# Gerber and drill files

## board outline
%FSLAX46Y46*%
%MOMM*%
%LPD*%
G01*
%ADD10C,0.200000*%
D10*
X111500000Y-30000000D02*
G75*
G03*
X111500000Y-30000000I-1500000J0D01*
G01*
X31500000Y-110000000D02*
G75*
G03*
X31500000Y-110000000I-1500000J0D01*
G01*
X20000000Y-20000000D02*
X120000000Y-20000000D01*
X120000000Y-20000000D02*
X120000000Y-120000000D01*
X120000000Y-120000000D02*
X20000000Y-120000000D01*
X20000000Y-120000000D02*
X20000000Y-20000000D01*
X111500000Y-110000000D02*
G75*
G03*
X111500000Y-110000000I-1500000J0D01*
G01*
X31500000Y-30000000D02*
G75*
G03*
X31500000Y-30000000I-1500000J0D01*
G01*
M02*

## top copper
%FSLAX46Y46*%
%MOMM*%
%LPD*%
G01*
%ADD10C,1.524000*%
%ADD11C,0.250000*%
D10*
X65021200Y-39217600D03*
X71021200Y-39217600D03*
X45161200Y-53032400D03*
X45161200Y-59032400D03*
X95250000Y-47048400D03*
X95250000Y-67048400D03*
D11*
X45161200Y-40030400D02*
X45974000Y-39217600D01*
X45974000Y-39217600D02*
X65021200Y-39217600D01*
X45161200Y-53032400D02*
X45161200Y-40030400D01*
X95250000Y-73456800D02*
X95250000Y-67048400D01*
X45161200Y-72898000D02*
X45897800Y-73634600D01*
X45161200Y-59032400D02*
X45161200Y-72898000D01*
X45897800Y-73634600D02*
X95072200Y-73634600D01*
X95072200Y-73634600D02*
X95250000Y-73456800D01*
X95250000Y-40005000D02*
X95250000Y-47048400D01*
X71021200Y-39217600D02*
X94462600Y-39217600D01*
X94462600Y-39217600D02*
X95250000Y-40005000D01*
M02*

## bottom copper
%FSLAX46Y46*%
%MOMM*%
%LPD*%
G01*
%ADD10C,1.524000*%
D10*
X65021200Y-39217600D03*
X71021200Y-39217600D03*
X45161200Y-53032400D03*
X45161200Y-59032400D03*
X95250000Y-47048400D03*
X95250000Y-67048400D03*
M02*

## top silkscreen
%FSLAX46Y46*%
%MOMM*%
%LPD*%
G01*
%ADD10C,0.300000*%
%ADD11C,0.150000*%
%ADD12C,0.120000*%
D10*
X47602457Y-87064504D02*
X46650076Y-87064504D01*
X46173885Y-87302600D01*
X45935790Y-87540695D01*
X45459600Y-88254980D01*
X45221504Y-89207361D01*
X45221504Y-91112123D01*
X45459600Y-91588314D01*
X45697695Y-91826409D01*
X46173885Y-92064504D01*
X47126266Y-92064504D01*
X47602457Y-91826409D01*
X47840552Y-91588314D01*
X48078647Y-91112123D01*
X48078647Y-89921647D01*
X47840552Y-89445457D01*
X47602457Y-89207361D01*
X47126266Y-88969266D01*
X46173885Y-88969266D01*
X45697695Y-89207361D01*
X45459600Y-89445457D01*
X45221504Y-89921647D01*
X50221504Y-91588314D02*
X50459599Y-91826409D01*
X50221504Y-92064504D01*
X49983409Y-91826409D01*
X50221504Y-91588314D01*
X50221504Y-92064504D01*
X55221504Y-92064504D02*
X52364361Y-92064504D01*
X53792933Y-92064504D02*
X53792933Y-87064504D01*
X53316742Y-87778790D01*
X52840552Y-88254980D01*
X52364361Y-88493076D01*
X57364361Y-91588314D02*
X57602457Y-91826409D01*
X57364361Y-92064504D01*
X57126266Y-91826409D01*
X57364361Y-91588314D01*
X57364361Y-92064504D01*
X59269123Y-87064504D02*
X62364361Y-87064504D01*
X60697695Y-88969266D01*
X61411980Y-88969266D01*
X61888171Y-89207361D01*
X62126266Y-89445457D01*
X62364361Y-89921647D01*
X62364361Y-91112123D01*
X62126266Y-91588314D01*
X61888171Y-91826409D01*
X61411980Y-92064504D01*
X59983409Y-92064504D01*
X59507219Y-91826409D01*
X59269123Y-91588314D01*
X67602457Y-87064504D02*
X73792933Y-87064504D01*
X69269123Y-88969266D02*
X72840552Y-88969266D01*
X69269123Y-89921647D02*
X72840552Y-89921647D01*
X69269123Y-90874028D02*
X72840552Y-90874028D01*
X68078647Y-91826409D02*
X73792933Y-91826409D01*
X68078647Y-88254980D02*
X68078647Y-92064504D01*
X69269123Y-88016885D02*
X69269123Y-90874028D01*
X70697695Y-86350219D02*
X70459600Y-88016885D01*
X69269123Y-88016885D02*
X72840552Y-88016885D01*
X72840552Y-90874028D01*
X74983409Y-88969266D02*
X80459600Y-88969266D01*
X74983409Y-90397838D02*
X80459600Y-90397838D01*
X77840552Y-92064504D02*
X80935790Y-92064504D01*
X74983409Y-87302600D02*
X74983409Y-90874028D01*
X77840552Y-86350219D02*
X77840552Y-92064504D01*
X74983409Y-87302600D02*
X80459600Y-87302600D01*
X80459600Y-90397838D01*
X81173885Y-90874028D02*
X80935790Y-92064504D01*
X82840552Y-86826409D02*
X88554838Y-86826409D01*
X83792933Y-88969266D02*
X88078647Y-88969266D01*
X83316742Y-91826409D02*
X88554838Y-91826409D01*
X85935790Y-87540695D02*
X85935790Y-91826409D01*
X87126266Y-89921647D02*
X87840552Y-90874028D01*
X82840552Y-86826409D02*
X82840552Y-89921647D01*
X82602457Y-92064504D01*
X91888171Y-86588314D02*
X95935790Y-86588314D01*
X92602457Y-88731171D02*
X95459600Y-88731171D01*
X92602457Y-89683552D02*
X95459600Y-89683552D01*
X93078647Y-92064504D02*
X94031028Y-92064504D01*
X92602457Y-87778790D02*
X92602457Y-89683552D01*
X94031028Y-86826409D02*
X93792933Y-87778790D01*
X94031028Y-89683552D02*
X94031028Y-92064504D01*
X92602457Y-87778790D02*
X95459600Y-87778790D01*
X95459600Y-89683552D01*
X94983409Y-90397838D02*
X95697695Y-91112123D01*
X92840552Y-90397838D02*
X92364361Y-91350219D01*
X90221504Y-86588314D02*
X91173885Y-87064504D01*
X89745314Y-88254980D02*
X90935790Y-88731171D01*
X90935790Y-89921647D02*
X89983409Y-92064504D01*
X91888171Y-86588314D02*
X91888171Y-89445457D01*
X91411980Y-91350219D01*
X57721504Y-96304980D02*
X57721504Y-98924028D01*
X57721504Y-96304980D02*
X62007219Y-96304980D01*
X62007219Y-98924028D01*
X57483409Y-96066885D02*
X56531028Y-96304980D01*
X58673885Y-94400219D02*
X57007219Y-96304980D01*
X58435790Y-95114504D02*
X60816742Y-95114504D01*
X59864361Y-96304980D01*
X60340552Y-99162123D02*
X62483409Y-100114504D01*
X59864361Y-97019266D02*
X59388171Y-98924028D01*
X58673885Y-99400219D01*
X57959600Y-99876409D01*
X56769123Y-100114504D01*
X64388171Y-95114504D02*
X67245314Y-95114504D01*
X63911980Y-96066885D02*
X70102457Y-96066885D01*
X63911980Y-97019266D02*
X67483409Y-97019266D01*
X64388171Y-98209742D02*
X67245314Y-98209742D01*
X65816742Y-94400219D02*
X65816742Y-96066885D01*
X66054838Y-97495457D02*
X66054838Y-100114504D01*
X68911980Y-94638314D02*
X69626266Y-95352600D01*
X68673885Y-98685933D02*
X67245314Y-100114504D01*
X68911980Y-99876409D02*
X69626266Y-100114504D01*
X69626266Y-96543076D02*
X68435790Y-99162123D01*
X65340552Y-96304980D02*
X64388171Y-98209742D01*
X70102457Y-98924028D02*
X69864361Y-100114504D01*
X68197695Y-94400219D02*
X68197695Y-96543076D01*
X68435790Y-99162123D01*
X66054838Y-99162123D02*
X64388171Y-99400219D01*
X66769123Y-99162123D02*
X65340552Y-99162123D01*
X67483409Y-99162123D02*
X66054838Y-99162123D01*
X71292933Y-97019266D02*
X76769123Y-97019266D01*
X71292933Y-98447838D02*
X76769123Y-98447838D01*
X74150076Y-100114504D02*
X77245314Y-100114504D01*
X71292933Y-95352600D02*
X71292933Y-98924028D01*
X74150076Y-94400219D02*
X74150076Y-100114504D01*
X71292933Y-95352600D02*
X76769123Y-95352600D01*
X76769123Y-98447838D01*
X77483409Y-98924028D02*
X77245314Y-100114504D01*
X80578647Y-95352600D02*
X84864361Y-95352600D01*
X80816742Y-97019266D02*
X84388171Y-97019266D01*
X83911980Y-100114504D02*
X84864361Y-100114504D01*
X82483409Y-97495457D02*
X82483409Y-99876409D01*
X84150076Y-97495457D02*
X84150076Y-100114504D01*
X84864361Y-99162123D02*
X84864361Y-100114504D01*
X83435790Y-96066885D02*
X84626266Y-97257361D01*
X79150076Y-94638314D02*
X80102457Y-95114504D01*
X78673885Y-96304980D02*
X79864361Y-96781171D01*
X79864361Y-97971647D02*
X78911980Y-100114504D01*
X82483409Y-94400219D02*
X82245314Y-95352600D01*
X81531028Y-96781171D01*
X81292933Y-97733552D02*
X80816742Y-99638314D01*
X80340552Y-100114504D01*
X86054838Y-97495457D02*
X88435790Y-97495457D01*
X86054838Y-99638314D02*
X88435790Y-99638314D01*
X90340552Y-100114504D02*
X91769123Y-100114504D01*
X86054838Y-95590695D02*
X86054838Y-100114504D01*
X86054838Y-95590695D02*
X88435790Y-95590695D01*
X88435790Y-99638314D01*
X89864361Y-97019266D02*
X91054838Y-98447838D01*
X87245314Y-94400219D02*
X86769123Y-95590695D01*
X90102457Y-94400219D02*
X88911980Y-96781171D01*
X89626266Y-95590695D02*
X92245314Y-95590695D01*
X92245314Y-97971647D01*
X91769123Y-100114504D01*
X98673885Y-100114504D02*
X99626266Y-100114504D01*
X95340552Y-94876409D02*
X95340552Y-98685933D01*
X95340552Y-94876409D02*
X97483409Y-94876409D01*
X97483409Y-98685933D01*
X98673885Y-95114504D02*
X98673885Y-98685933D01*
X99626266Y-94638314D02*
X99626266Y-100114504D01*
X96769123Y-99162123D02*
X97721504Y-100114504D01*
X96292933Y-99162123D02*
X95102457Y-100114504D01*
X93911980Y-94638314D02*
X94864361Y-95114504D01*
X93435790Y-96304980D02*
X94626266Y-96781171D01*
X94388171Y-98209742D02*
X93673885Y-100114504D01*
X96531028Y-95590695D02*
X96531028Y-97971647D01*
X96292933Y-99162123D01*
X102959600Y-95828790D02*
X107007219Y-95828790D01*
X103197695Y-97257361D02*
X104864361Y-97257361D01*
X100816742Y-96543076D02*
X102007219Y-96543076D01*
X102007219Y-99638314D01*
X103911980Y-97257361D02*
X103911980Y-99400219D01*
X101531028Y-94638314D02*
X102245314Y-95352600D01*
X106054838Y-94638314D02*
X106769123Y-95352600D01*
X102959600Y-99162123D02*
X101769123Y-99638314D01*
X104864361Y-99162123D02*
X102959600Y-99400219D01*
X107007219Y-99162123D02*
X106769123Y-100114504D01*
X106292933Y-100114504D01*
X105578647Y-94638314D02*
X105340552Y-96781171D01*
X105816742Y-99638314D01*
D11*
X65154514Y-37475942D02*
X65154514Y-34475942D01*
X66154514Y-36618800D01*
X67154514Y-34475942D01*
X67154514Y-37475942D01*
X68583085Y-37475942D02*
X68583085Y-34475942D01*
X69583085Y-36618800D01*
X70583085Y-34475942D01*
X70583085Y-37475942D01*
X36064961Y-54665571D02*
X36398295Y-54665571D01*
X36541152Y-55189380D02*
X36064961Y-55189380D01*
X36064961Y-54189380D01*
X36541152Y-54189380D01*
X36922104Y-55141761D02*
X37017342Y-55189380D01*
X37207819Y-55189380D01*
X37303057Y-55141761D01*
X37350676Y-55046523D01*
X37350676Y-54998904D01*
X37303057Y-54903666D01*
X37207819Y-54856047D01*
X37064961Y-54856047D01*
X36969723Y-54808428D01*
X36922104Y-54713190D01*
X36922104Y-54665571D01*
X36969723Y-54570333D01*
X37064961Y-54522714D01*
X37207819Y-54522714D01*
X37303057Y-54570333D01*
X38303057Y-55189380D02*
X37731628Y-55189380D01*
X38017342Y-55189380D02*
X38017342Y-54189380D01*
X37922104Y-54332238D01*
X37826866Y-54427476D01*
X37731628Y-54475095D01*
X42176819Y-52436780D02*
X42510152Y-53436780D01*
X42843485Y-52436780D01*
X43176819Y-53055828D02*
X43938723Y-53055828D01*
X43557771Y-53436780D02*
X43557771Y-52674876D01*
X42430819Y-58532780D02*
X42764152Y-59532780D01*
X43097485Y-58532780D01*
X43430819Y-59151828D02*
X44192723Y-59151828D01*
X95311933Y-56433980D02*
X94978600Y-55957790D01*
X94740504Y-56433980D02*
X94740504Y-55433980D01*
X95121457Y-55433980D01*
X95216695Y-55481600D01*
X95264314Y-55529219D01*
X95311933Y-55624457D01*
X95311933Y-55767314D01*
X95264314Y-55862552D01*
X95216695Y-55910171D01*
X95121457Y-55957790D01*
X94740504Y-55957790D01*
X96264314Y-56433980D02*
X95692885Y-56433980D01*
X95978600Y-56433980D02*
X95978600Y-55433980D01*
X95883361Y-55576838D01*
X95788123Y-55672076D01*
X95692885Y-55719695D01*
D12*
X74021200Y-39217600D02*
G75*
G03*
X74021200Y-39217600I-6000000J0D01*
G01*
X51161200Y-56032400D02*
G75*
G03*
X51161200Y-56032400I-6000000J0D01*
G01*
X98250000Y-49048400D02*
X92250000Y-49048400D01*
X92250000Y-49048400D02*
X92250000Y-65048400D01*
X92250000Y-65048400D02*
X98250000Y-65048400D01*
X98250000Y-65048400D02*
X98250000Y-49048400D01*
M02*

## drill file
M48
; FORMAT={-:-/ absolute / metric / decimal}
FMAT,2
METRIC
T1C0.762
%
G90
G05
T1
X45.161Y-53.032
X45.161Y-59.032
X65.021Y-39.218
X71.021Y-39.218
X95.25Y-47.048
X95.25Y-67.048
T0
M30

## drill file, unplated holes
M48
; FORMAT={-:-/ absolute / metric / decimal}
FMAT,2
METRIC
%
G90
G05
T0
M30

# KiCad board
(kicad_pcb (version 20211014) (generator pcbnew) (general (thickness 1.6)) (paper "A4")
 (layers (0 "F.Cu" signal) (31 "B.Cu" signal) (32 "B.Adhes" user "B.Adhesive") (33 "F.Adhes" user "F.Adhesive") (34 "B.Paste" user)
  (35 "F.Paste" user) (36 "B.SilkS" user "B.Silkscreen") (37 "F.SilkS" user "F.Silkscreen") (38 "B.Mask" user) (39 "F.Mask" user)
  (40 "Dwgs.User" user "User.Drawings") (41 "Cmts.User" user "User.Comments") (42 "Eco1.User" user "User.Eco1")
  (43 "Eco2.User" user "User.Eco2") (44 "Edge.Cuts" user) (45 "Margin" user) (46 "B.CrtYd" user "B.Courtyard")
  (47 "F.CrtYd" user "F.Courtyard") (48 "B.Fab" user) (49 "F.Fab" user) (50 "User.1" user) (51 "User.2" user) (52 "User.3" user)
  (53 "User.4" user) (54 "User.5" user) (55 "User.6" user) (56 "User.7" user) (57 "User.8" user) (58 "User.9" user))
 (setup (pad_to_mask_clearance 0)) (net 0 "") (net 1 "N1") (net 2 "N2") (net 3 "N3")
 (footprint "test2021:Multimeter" (layer "F.Cu") (at 68.0212 39.2176 90)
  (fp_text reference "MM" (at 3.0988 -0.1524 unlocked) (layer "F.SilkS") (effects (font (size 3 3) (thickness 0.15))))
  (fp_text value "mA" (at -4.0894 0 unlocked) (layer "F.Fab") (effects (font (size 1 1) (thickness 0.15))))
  (fp_circle (center 0 0) (end 6 0) (layer "F.SilkS") (width 0.12) (fill none))
  (pad "1" thru_hole circle (at 0 -3 90) (size 1.524 1.524) (drill 0.762) (layers *.Cu *.Mask) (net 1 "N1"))
  (pad "2" thru_hole circle (at 0 3 90) (size 1.524 1.524) (drill 0.762) (layers *.Cu *.Mask) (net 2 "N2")))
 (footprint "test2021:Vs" (layer "F.Cu") (at 45.1612 56.0324)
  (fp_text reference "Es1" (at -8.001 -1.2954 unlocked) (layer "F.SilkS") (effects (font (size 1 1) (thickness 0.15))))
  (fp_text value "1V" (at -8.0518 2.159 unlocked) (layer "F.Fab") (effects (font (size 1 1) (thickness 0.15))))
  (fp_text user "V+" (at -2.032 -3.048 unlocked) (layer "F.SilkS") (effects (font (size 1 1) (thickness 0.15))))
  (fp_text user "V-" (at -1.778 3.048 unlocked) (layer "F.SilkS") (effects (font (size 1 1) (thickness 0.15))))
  (fp_circle (center 0 0) (end 6 0) (layer "F.SilkS") (width 0.12) (fill none))
  (pad "1" thru_hole circle (at 0 -3) (size 1.524 1.524) (drill 0.762) (layers *.Cu *.Mask) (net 1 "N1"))
  (pad "2" thru_hole circle (at 0 3) (size 1.524 1.524) (drill 0.762) (layers *.Cu *.Mask) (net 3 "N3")))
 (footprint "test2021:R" (layer "F.Cu") (at 95.25 57.0484 -90)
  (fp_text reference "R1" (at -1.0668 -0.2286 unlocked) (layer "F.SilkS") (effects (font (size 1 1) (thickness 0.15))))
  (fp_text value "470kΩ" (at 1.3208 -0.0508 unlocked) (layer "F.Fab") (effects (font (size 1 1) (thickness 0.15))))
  (fp_rect (start -8 -3) (end 8 3) (layer "F.SilkS") (width 0.12) (fill none))
  (pad "1" thru_hole circle (at -10 0 270) (size 1.524 1.524) (drill 0.762) (layers *.Cu *.Mask) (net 2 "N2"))
  (pad "2" thru_hole circle (at 10 0 270) (size 1.524 1.524) (drill 0.762) (layers *.Cu *.Mask) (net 3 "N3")))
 (gr_circle (center 110 30) (end 111.5 30) (layer "Edge.Cuts") (width 0.2) (fill none))
 (gr_circle (center 30 110) (end 31.5 110) (layer "Edge.Cuts") (width 0.2) (fill none))
 (gr_rect (start 20 20) (end 120 120) (layer "Edge.Cuts") (width 0.2) (fill none))
 (gr_circle (center 110 110) (end 111.5 110) (layer "Edge.Cuts") (width 0.2) (fill none))
 (gr_circle (center 30 30) (end 31.5 30) (layer "Edge.Cuts") (width 0.2) (fill none))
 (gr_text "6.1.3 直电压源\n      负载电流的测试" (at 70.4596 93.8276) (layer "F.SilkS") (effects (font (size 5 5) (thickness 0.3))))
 (segment (start 45.1612 40.0304) (end 45.974 39.2176) (width 0.25) (layer "F.Cu") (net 1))
 (segment (start 45.974 39.2176) (end 65.0212 39.2176) (width 0.25) (layer "F.Cu") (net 1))
 (segment (start 45.1612 53.0324) (end 45.1612 40.0304) (width 0.25) (layer "F.Cu") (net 1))
 (segment (start 95.25 73.4568) (end 95.25 67.0484) (width 0.25) (layer "F.Cu") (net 3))
 (segment (start 45.1612 72.898) (end 45.8978 73.6346) (width 0.25) (layer "F.Cu") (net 3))
 (segment (start 45.1612 59.0324) (end 45.1612 72.898) (width 0.25) (layer "F.Cu") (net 3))
 (segment (start 45.8978 73.6346) (end 95.0722 73.6346) (width 0.25) (layer "F.Cu") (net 3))
 (segment (start 95.0722 73.6346) (end 95.25 73.4568) (width 0.25) (layer "F.Cu") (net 3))
 (segment (start 95.25 40.005) (end 95.25 47.0484) (width 0.25) (layer "F.Cu") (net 2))
 (segment (start 71.0212 39.2176) (end 94.4626 39.2176) (width 0.25) (layer "F.Cu") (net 2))
 (segment (start 94.4626 39.2176) (end 95.25 40.005) (width 0.25) (layer "F.Cu") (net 2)))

